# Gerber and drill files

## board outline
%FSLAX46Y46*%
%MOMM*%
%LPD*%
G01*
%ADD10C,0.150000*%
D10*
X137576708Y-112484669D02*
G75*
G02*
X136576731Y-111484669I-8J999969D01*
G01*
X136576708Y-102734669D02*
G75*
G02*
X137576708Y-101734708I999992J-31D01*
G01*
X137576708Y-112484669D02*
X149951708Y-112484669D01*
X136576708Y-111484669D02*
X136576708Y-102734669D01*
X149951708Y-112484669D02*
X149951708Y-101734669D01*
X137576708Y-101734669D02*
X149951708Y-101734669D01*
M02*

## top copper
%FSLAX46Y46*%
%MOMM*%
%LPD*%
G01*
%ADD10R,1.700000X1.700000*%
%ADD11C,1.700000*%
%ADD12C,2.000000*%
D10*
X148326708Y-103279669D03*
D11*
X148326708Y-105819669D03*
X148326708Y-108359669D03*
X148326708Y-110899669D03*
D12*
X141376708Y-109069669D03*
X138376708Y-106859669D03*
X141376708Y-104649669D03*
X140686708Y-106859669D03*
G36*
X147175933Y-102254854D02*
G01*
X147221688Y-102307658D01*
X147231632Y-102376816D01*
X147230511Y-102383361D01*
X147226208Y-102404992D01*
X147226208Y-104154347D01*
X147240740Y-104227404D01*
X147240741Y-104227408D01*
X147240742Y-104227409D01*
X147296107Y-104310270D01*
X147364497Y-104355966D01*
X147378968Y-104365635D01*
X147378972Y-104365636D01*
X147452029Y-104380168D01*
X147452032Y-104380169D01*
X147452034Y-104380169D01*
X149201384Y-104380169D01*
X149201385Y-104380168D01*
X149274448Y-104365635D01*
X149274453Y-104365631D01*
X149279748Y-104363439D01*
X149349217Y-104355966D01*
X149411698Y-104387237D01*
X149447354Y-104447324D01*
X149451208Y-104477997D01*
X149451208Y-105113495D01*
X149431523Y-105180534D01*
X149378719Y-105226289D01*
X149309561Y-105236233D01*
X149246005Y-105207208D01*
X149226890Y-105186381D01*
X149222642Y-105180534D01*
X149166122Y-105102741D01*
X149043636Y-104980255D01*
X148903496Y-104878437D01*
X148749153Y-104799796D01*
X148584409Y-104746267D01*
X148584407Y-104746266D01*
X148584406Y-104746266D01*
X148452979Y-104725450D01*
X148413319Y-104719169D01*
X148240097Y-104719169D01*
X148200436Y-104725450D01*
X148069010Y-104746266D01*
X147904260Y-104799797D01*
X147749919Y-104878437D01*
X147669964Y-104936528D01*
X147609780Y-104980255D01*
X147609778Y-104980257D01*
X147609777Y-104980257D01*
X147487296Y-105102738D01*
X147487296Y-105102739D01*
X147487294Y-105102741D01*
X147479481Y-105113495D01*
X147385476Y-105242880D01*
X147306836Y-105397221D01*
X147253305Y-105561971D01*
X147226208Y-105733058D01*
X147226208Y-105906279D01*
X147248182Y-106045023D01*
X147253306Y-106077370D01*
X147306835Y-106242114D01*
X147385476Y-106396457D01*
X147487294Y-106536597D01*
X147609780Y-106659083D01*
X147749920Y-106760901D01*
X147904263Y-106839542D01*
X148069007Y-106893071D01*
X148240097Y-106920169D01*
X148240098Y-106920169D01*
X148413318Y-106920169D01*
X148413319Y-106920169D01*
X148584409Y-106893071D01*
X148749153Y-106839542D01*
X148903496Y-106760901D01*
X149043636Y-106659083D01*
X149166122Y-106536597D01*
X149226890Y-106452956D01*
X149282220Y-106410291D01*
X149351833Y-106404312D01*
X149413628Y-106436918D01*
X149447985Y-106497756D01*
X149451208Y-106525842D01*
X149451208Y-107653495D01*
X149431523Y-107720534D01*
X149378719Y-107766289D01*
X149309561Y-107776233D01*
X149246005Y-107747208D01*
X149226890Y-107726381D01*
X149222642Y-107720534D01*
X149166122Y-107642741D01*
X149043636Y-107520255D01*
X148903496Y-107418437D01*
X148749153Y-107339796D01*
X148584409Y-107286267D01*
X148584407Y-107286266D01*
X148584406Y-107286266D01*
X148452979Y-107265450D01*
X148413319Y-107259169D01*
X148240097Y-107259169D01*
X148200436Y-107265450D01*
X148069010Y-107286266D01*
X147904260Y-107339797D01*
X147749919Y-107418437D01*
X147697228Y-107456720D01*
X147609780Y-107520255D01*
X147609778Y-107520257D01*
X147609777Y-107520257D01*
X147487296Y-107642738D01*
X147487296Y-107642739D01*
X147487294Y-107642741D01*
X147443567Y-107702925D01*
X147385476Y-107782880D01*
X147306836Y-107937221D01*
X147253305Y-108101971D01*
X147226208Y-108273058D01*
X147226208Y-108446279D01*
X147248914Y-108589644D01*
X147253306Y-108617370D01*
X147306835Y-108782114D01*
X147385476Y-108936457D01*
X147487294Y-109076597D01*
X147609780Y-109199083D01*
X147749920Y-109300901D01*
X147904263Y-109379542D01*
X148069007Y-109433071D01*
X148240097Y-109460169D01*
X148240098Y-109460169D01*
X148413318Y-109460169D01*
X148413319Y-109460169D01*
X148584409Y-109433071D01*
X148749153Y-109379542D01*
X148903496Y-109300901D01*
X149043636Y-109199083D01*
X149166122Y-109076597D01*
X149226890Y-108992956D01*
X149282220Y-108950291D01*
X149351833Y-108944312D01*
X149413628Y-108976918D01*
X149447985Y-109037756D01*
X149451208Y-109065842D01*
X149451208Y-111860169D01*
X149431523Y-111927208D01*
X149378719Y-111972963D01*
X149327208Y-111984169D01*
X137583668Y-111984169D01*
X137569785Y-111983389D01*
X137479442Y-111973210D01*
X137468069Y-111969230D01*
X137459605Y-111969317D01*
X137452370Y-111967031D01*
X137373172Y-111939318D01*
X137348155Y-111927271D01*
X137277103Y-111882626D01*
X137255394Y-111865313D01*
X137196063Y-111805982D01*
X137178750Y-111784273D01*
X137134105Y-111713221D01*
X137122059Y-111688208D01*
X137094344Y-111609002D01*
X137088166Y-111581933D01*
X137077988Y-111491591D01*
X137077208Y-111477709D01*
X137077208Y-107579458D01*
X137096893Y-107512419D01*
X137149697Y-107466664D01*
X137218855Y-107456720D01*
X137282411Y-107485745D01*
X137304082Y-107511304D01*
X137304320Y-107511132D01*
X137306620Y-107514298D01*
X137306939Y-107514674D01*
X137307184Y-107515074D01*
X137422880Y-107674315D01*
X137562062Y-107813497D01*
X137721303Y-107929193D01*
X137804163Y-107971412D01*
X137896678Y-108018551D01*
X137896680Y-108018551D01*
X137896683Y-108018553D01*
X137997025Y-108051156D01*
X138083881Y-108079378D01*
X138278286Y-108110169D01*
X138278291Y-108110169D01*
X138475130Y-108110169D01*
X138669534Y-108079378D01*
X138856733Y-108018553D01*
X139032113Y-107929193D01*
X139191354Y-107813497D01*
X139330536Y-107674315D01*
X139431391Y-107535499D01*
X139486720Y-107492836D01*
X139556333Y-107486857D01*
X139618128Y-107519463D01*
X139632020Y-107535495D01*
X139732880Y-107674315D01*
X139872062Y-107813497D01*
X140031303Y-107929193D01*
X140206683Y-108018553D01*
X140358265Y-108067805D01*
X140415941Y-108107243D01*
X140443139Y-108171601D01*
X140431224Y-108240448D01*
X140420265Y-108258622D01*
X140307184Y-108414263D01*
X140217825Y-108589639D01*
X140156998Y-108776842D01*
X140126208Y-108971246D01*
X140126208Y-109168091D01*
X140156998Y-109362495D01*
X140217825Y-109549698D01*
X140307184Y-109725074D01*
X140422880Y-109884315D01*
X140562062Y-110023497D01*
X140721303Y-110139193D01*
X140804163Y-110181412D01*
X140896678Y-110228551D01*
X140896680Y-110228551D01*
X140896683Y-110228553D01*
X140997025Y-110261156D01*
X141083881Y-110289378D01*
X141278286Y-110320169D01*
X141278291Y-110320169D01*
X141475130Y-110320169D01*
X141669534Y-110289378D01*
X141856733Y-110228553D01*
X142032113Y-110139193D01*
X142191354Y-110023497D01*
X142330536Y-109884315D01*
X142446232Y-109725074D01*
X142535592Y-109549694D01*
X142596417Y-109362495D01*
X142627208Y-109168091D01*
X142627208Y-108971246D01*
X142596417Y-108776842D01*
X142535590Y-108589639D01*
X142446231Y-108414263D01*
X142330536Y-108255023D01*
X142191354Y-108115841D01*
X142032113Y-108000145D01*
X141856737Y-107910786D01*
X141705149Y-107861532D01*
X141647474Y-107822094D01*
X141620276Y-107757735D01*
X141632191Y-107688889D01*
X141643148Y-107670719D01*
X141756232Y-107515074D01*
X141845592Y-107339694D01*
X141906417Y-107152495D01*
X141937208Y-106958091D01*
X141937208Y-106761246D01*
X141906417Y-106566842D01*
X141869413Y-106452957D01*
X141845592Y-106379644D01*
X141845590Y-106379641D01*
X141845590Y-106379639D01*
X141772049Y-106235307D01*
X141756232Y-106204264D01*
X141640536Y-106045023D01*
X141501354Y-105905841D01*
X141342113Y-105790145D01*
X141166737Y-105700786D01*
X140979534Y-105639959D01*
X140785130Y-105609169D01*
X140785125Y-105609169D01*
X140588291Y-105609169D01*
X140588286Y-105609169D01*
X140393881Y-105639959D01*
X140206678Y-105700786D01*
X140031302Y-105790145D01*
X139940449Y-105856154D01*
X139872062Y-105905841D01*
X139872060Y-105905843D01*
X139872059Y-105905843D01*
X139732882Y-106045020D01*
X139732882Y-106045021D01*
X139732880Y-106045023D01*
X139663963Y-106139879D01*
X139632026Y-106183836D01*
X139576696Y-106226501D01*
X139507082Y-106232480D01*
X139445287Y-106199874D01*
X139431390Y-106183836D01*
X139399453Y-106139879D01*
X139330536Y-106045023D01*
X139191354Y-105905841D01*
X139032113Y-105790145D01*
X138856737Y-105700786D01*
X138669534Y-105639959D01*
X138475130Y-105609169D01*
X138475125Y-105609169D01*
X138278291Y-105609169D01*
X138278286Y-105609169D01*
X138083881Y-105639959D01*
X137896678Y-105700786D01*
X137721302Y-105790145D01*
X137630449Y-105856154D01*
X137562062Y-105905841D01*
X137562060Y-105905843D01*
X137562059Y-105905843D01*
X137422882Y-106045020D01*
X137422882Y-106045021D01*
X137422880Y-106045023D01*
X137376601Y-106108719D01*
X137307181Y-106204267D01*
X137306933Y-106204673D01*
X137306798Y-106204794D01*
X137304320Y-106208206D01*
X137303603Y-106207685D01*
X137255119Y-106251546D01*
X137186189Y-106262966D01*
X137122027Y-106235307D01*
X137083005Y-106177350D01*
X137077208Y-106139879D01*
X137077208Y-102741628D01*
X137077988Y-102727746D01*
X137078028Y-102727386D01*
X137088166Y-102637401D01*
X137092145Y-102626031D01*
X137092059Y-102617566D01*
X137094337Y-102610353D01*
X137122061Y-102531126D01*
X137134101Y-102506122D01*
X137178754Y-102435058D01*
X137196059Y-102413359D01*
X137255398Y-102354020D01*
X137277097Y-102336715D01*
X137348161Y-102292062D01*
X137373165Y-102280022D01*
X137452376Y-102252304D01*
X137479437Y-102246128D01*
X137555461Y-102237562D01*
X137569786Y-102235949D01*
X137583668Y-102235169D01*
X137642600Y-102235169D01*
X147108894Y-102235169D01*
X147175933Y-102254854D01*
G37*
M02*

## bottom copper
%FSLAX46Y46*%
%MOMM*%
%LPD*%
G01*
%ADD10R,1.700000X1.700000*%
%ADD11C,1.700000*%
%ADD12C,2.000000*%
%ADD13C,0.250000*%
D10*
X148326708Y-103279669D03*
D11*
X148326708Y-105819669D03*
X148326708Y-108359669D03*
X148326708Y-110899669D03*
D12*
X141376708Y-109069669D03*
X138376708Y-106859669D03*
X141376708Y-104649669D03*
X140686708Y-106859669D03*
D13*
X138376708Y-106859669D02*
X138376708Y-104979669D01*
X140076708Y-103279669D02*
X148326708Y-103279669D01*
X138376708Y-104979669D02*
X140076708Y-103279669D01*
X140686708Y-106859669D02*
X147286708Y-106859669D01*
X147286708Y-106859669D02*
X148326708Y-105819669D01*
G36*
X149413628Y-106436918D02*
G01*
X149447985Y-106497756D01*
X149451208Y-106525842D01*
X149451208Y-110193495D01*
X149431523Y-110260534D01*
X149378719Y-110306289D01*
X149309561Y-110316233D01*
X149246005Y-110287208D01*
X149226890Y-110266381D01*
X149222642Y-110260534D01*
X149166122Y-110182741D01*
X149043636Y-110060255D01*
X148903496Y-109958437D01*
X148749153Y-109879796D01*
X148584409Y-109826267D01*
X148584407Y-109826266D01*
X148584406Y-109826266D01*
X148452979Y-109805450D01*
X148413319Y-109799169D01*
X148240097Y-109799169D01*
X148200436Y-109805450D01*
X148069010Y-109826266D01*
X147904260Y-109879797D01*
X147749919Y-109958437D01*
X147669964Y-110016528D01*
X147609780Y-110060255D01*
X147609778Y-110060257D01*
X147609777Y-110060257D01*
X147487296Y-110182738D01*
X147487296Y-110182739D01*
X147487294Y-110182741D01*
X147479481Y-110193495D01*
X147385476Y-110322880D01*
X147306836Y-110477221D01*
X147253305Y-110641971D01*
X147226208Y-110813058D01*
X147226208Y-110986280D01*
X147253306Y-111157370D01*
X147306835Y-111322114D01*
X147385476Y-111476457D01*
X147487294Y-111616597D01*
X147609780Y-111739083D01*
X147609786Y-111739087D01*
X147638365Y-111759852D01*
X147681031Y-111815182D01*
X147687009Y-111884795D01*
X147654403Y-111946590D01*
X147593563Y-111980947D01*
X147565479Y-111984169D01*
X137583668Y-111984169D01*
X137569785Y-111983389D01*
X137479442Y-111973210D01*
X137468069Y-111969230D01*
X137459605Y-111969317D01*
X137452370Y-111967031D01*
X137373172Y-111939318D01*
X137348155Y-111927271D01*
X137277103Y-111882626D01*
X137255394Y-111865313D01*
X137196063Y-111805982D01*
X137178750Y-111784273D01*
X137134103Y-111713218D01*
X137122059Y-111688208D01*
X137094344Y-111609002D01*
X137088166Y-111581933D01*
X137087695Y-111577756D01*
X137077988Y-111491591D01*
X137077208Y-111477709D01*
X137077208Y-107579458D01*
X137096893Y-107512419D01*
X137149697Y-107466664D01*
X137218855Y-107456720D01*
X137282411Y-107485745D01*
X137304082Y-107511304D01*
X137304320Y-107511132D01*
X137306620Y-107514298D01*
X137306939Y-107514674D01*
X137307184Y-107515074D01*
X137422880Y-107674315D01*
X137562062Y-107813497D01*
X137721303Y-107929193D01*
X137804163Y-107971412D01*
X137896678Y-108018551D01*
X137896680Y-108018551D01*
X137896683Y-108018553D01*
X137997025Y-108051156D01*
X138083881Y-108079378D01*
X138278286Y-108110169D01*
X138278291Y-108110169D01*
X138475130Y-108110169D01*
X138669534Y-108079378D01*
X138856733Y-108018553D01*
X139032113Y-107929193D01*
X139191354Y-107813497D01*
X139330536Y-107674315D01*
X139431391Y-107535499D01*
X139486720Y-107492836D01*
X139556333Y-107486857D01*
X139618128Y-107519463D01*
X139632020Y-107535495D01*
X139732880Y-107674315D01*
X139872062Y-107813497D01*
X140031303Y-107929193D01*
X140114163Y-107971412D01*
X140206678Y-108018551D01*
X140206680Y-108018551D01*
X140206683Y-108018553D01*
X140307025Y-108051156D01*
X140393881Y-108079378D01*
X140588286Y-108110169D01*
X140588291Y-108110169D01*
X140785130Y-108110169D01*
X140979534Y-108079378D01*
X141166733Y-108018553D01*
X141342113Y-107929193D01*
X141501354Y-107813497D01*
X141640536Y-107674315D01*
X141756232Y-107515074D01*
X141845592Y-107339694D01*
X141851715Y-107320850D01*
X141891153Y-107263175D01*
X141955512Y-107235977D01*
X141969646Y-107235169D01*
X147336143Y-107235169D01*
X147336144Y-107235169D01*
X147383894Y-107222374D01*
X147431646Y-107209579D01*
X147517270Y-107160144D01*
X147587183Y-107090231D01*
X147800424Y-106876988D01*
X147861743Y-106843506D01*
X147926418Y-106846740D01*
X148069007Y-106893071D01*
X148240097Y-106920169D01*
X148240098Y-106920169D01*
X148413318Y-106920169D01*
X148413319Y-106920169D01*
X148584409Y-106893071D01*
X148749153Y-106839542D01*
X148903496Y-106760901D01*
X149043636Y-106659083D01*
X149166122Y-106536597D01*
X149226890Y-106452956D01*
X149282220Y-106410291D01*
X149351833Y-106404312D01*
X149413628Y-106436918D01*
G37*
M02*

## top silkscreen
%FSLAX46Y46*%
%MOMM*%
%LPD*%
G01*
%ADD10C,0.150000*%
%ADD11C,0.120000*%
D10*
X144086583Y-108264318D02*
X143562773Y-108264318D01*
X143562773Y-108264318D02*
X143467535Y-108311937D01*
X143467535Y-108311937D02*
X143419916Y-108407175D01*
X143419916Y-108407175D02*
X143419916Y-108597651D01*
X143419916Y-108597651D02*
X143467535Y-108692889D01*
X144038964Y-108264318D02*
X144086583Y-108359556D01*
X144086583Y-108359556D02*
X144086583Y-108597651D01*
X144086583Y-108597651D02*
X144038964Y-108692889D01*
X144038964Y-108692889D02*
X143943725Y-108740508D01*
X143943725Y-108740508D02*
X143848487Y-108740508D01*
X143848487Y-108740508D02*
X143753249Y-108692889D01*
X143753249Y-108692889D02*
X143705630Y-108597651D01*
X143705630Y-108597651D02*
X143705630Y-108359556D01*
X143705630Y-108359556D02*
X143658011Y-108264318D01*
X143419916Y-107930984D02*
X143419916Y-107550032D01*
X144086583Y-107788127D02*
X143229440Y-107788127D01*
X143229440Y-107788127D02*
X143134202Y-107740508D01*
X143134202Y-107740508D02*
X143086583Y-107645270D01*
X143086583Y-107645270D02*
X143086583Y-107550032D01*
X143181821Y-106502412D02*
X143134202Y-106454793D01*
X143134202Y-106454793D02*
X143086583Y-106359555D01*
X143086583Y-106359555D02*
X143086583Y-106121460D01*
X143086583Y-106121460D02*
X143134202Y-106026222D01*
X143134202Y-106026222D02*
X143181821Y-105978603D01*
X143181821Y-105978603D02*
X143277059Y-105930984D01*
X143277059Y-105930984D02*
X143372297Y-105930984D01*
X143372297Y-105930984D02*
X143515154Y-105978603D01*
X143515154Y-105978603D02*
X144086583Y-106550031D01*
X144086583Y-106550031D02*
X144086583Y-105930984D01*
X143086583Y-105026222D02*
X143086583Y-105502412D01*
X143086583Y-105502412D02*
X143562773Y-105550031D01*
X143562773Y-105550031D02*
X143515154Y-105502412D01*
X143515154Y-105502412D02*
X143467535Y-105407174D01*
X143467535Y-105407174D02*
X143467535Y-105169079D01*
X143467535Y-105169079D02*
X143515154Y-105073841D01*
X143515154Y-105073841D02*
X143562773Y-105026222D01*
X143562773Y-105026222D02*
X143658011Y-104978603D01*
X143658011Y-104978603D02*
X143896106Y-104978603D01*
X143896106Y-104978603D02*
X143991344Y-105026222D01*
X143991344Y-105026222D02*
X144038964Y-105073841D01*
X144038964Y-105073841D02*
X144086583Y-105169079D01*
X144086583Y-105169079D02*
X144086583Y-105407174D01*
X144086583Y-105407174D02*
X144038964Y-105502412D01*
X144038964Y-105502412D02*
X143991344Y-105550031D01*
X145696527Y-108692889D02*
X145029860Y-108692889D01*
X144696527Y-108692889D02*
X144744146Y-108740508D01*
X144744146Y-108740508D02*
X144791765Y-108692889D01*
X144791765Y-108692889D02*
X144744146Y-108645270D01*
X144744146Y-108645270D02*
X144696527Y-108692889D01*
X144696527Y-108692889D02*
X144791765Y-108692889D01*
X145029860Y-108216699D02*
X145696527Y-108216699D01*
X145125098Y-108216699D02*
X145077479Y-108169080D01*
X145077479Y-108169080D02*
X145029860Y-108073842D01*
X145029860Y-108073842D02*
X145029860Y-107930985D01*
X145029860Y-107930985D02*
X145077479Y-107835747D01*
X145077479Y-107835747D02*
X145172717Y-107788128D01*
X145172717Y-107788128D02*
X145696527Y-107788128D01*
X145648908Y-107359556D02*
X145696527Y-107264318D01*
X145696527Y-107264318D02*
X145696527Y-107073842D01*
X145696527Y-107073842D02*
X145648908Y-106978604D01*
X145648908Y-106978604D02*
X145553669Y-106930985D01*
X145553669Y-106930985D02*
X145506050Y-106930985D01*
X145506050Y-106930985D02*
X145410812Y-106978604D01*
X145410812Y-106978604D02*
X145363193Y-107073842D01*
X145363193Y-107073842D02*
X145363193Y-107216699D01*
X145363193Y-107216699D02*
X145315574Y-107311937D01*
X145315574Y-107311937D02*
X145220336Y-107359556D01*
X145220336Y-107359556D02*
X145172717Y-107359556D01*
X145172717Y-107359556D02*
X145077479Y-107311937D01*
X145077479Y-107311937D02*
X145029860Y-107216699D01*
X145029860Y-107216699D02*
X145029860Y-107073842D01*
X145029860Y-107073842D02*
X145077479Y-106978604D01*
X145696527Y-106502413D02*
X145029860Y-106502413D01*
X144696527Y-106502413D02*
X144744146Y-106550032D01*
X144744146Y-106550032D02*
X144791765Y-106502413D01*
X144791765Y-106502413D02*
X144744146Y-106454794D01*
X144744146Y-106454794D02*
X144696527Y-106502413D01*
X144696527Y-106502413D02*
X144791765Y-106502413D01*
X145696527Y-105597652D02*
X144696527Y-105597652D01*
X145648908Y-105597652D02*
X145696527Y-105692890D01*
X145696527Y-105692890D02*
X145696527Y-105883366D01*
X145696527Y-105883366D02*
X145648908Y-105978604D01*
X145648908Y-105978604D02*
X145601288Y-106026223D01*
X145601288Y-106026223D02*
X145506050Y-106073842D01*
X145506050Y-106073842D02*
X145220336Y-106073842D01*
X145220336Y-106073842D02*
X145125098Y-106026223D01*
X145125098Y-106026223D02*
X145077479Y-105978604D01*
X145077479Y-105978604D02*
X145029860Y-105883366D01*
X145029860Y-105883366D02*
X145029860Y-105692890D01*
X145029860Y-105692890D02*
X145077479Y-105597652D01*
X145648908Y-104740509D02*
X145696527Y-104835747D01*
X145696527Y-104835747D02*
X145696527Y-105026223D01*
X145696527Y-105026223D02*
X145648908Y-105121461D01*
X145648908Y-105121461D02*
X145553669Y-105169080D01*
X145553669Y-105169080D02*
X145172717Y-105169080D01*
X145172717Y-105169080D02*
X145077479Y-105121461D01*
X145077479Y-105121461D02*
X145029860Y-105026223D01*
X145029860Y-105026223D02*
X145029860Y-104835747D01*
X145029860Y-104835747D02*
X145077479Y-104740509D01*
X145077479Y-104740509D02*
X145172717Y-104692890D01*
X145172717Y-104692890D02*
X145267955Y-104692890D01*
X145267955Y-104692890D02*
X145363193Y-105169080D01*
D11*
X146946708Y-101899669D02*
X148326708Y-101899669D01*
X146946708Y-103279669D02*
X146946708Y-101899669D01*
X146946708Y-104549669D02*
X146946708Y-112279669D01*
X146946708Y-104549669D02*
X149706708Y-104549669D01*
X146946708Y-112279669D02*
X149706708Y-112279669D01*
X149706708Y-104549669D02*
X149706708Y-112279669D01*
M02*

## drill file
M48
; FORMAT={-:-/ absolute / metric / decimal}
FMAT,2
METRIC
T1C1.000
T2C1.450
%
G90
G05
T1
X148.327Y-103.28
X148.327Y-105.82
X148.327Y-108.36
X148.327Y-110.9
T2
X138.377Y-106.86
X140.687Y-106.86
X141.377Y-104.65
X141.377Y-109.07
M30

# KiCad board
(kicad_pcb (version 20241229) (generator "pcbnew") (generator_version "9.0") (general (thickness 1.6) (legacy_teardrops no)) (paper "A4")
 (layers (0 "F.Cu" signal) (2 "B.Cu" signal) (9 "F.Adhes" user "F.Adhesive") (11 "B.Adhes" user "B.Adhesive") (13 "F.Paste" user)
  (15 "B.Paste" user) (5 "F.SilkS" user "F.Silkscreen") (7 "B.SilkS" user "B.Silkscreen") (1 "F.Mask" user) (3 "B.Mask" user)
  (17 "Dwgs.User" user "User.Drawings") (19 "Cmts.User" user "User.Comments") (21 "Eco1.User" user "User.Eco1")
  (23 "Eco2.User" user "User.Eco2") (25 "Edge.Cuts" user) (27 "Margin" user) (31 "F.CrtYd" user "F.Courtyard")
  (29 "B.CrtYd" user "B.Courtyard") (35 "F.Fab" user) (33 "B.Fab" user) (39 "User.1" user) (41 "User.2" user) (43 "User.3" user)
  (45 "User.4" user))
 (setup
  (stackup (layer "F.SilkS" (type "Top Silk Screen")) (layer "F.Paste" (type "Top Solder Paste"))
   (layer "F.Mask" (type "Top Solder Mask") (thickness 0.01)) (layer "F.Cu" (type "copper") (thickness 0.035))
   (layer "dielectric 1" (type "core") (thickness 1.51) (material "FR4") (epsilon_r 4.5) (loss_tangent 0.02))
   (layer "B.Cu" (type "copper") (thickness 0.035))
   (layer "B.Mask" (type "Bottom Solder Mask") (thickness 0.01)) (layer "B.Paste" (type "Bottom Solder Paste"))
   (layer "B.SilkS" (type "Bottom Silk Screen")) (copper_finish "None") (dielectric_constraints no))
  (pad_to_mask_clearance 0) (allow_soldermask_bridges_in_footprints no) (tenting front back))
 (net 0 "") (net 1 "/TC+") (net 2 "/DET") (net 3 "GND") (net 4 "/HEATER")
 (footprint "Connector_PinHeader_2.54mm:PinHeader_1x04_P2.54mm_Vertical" (layer "F.Cu") (at 148.326708 103.279669)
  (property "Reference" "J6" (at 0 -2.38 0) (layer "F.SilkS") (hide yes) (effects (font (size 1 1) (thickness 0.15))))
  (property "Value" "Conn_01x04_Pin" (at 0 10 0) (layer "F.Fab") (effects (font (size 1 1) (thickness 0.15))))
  (fp_line (start -1.38 -1.38) (end 0 -1.38) (stroke (width 0.12) (type solid)) (layer "F.SilkS"))
  (fp_line (start -1.38 0) (end -1.38 -1.38) (stroke (width 0.12) (type solid)) (layer "F.SilkS"))
  (fp_line (start -1.38 1.27) (end -1.38 9) (stroke (width 0.12) (type solid)) (layer "F.SilkS"))
  (fp_line (start -1.38 1.27) (end 1.38 1.27) (stroke (width 0.12) (type solid)) (layer "F.SilkS"))
  (fp_line (start -1.38 9) (end 1.38 9) (stroke (width 0.12) (type solid)) (layer "F.SilkS"))
  (fp_line (start 1.38 1.27) (end 1.38 9) (stroke (width 0.12) (type solid)) (layer "F.SilkS"))
  (pad "1" thru_hole rect (at 0 0) (size 1.7 1.7) (drill 1) (layers "*.Cu" "*.Mask") (remove_unused_layers no) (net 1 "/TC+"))
  (pad "2" thru_hole circle (at 0 2.54) (size 1.7 1.7) (drill 1) (layers "*.Cu" "*.Mask") (remove_unused_layers no) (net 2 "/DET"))
  (pad "3" thru_hole circle (at 0 5.08) (size 1.7 1.7) (drill 1) (layers "*.Cu" "*.Mask") (remove_unused_layers no) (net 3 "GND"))
  (pad "4" thru_hole circle (at 0 7.62) (size 1.7 1.7) (drill 1) (layers "*.Cu" "*.Mask") (remove_unused_layers no) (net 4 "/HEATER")))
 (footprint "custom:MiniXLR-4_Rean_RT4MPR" (layer "B.Cu") (at 140.686708 106.859669 90)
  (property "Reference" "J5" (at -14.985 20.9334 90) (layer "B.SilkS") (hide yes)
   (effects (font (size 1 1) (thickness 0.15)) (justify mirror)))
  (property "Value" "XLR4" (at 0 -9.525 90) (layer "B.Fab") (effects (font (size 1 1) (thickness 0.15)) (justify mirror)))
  (pad "1" thru_hole circle (at -2.21 0.69 270) (size 2 2) (drill 1.45) (layers "*.Cu" "*.Mask") (remove_unused_layers no) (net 3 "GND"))
  (pad "2" thru_hole circle (at 0 -2.31 270) (size 2 2) (drill 1.45) (layers "*.Cu" "*.Mask") (remove_unused_layers no) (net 1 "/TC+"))
  (pad "3" thru_hole circle (at 2.21 0.69 270) (size 2 2) (drill 1.45) (layers "*.Cu" "*.Mask") (remove_unused_layers no) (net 4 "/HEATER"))
  (pad "4" thru_hole circle (at 0 0 270) (size 2 2) (drill 1.45) (layers "*.Cu" "*.Mask") (remove_unused_layers no) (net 2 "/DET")))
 (gr_arc (start 137.576708 112.484669) (mid 136.869601 112.191776) (end 136.576708 111.484669) (stroke (width 0.15) (type default))
  (layer "Edge.Cuts"))
 (gr_arc (start 136.576708 102.734669) (mid 136.869601 102.027562) (end 137.576708 101.734669) (stroke (width 0.15) (type default))
  (layer "Edge.Cuts"))
 (gr_line (start 137.576708 112.484669) (end 149.951708 112.484669) (stroke (width 0.15) (type default)) (layer "Edge.Cuts"))
 (gr_line (start 136.576708 111.484669) (end 136.576708 102.734669) (stroke (width 0.15) (type default)) (layer "Edge.Cuts"))
 (gr_line (start 149.951708 112.484669) (end 149.951708 101.734669) (stroke (width 0.15) (type default)) (layer "Edge.Cuts"))
 (gr_line (start 137.576708 101.734669) (end 149.951708 101.734669) (stroke (width 0.15) (type default)) (layer "Edge.Cuts"))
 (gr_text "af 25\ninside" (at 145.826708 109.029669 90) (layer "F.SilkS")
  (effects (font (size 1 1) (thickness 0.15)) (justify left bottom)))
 (segment (start 138.376708 106.859669) (end 138.376708 104.979669) (width 0.25) (layer "B.Cu") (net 1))
 (segment (start 140.076708 103.279669) (end 148.326708 103.279669) (width 0.25) (layer "B.Cu") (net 1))
 (segment (start 138.376708 104.979669) (end 140.076708 103.279669) (width 0.25) (layer "B.Cu") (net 1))
 (segment (start 140.686708 106.859669) (end 147.286708 106.859669) (width 0.25) (layer "B.Cu") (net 2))
 (segment (start 147.286708 106.859669) (end 148.326708 105.819669) (width 0.25) (layer "B.Cu") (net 2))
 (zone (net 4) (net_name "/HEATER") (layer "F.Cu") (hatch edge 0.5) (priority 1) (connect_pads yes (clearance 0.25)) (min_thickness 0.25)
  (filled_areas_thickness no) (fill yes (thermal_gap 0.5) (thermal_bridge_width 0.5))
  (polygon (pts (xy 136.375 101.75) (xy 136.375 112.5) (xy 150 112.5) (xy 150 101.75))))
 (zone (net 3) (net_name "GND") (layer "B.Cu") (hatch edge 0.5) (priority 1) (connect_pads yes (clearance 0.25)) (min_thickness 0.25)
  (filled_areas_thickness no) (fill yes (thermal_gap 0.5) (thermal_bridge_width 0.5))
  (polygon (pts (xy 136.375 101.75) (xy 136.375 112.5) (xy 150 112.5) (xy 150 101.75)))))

